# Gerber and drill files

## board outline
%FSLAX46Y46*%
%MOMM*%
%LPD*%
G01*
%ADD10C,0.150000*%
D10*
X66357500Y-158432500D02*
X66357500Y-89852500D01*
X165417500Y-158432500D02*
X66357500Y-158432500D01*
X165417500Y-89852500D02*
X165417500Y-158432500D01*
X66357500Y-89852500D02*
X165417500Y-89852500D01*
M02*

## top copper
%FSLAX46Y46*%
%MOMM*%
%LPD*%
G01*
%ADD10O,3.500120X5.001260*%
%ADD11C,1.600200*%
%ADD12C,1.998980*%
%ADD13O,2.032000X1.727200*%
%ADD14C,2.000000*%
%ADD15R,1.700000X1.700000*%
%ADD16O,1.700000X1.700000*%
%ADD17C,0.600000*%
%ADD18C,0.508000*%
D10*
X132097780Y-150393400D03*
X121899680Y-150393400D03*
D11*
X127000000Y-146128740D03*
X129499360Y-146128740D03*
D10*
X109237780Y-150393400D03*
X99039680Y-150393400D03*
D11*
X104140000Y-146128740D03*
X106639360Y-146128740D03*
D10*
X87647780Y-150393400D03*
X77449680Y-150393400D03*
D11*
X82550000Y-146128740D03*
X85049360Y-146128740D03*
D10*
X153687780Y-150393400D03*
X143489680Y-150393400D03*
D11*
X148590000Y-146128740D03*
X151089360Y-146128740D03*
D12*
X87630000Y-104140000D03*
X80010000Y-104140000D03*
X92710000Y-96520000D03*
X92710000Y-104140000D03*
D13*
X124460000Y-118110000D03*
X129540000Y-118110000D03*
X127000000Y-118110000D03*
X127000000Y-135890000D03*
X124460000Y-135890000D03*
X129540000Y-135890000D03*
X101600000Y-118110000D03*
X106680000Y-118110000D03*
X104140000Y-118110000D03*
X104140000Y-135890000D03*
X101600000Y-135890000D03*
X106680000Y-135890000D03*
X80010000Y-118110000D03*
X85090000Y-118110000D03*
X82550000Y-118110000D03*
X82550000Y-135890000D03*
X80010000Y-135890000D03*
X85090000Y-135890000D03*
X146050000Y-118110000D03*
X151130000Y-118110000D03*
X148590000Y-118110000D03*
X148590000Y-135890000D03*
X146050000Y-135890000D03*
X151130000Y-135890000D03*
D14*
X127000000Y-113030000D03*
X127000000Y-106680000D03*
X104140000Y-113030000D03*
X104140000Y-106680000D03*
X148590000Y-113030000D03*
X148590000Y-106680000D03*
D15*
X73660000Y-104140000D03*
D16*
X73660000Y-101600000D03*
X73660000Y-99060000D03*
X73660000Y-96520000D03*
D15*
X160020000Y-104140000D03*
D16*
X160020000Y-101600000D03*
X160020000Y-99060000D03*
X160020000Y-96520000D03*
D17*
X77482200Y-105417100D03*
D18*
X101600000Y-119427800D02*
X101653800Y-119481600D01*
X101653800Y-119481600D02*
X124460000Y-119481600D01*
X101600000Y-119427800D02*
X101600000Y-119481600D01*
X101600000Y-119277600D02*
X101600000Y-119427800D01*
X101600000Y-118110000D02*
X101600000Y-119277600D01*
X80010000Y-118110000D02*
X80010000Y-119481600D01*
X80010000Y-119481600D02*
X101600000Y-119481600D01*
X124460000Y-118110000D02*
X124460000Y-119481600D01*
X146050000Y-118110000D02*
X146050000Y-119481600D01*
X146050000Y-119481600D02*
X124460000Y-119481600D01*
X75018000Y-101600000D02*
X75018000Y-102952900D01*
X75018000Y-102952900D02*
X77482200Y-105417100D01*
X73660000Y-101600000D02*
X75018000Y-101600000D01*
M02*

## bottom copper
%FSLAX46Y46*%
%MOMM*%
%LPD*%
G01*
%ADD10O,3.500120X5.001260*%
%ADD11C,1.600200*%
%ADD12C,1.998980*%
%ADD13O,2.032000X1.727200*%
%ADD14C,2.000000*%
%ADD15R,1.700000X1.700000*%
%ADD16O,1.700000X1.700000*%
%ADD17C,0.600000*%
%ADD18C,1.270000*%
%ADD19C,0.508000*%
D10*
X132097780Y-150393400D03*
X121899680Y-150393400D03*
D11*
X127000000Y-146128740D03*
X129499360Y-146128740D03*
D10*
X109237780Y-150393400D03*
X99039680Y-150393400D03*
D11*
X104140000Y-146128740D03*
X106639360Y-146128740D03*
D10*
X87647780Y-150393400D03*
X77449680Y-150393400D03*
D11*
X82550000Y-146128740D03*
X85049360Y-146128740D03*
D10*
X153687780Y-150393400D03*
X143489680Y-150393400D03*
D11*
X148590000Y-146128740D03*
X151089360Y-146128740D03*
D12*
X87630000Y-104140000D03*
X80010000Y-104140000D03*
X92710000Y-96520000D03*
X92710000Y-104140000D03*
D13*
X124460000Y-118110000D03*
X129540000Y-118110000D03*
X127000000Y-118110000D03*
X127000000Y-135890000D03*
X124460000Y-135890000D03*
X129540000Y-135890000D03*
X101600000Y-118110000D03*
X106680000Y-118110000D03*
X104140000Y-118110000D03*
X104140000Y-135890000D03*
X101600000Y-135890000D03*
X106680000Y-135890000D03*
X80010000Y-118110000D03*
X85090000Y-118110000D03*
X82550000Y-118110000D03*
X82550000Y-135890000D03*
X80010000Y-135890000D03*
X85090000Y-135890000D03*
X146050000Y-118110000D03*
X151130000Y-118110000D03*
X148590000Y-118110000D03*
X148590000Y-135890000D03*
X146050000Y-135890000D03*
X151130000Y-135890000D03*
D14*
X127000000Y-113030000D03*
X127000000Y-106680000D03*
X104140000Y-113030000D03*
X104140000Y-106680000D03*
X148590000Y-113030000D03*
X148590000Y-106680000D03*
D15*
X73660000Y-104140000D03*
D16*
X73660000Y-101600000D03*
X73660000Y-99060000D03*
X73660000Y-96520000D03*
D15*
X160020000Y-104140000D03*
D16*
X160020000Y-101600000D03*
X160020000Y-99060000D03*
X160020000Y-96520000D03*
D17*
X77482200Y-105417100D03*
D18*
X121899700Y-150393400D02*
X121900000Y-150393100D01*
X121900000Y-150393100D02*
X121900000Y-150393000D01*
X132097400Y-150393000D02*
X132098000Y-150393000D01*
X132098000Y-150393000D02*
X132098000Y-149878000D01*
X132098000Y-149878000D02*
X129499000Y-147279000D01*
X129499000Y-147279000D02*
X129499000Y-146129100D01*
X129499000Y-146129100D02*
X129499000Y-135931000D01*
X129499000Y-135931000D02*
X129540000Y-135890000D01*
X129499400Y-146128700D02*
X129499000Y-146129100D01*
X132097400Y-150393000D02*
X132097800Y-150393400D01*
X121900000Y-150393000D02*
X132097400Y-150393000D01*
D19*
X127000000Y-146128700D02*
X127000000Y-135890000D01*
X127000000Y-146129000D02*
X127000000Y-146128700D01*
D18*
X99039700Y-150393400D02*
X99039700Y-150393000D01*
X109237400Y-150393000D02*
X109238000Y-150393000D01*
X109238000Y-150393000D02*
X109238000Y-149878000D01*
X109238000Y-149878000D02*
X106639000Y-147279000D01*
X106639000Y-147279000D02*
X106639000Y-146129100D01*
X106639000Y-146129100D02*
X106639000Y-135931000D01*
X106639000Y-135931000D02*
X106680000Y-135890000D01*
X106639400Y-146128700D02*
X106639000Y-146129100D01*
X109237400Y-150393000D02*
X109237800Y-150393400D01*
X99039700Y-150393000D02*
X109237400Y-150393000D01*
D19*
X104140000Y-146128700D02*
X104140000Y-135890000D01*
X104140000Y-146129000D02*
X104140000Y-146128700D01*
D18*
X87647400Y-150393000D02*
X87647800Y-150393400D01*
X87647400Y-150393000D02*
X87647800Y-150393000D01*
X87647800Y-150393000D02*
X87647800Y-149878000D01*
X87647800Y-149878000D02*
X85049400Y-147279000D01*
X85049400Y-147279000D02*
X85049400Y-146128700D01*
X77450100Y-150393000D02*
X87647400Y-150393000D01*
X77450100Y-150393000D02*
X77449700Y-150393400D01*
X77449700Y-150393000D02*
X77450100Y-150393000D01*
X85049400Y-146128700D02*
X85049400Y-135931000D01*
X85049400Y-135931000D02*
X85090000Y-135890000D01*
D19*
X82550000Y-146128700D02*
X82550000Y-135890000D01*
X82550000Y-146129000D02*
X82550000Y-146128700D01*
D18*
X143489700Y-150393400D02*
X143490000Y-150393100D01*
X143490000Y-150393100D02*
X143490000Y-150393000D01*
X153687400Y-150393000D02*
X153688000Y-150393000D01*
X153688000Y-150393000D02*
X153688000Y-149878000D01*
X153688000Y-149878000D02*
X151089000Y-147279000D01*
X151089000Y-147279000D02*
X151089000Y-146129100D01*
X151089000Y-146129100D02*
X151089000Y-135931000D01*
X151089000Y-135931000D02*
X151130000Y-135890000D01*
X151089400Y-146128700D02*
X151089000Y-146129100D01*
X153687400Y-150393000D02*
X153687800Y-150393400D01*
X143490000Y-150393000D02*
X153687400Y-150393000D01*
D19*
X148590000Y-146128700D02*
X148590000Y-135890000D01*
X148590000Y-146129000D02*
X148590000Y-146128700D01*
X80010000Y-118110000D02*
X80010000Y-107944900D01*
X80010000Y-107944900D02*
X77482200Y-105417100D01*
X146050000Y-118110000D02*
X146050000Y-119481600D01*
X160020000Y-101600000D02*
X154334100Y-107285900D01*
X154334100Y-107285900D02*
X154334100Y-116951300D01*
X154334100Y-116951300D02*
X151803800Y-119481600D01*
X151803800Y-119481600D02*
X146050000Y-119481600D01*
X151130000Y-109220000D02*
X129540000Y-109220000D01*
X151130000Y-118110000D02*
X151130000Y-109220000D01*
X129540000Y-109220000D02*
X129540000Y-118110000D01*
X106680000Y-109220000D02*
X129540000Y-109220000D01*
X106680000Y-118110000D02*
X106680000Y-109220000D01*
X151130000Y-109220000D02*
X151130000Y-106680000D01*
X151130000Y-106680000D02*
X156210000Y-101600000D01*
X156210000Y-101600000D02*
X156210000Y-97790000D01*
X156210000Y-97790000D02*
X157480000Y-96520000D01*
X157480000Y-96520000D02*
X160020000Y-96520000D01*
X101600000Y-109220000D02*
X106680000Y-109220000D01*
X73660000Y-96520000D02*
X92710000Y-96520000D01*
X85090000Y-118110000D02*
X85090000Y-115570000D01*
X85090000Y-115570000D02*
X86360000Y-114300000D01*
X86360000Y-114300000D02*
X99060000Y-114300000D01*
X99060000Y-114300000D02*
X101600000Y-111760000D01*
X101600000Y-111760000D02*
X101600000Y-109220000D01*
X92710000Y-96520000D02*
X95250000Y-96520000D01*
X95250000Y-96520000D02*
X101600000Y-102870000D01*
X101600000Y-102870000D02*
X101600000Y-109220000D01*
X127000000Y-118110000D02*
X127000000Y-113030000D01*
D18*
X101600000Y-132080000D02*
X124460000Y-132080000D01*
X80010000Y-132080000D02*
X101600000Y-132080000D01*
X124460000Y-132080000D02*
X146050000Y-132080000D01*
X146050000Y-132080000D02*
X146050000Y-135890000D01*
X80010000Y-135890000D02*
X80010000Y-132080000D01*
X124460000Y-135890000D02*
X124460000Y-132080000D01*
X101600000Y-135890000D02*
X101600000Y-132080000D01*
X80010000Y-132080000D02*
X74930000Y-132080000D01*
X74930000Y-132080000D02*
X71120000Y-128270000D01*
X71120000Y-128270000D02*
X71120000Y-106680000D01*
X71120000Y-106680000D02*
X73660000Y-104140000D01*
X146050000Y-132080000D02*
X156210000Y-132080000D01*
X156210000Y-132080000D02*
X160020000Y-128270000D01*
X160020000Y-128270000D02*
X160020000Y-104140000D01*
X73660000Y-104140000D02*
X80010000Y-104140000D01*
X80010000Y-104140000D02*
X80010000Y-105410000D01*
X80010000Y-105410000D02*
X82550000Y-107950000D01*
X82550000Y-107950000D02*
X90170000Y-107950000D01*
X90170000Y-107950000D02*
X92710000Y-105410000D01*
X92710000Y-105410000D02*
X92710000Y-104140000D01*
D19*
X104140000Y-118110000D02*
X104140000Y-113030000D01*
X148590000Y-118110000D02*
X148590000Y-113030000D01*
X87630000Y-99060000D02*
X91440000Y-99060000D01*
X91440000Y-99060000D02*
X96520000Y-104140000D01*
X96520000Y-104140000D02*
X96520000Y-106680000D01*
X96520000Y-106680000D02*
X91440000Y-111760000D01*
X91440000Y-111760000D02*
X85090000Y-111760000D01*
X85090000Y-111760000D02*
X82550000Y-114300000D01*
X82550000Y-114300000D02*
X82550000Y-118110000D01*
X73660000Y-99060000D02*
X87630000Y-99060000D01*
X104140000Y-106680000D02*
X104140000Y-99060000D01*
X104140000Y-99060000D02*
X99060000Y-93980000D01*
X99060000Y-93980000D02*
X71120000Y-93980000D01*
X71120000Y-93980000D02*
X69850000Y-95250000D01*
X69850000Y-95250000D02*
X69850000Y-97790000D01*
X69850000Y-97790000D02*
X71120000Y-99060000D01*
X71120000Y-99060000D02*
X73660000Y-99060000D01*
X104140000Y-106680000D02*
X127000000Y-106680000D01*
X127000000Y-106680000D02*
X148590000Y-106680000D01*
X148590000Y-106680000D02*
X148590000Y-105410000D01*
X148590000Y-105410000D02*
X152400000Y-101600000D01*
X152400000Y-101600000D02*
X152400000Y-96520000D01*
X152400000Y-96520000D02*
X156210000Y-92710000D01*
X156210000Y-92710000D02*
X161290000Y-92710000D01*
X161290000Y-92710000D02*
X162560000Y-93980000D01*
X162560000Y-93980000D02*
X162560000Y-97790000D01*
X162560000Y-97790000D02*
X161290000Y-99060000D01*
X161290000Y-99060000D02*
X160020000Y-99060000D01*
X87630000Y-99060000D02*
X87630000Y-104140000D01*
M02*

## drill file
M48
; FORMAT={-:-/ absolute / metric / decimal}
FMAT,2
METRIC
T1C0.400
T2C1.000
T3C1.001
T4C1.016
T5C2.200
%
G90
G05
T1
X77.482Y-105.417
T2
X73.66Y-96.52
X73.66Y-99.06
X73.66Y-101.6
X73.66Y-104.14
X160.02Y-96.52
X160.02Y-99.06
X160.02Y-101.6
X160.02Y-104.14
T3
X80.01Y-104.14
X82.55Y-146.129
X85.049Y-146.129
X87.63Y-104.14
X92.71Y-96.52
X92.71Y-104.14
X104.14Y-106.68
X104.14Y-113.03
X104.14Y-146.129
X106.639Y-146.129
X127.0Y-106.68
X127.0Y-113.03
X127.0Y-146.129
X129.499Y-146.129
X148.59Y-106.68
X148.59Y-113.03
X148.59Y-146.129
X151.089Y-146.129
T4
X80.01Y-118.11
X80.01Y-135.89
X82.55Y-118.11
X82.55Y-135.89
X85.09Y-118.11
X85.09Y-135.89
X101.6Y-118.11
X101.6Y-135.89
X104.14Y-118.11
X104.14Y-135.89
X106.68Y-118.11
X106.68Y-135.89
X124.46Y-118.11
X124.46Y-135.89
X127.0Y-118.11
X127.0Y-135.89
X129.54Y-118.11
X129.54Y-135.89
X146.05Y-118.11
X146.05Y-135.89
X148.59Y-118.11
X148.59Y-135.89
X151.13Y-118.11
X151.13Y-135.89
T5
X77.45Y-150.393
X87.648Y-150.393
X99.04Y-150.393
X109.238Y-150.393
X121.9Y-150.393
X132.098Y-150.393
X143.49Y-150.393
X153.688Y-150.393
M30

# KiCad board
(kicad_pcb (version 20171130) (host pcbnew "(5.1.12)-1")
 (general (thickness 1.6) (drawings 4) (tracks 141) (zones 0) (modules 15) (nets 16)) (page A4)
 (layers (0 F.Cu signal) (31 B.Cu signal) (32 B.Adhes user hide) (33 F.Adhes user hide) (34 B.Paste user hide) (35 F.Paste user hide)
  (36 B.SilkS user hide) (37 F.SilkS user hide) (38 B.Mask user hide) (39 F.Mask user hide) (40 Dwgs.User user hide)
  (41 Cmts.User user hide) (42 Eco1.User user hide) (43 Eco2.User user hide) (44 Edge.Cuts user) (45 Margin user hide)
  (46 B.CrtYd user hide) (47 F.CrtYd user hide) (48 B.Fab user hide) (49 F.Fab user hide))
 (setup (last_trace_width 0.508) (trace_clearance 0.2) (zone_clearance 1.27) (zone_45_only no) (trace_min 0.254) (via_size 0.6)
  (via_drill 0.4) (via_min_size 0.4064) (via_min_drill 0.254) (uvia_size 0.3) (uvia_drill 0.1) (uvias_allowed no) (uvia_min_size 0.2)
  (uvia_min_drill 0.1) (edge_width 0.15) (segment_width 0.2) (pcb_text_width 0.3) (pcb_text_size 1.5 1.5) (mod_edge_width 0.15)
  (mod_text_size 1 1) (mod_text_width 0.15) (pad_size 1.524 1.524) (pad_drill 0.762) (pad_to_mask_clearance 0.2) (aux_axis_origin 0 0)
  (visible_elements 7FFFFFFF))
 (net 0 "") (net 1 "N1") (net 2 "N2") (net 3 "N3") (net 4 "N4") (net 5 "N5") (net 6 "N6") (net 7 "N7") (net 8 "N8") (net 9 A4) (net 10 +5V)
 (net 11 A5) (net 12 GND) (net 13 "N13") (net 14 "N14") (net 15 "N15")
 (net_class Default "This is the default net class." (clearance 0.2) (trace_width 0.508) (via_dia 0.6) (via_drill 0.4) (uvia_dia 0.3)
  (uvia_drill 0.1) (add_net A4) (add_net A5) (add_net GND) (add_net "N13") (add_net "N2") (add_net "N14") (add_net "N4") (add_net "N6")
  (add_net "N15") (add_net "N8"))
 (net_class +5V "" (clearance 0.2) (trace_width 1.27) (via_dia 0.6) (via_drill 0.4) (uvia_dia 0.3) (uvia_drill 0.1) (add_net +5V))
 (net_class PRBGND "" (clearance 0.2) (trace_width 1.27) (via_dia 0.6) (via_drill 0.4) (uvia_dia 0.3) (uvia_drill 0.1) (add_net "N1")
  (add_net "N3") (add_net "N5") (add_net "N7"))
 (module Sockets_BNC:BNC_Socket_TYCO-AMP (layer F.Cu) (at 127 151.13 180)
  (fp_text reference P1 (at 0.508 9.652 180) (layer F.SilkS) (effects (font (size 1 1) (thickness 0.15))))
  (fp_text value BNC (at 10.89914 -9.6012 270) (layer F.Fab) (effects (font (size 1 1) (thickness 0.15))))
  (pad 2 thru_hole oval (at -5.09778 0.7366 180) (size 3.50012 5.00126) (drill 2.19964) (layers *.Cu *.Mask) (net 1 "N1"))
  (pad 2 thru_hole oval (at 5.10032 0.7366 180) (size 3.50012 5.00126) (drill 2.19964) (layers *.Cu *.Mask) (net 1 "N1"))
  (pad 1 thru_hole circle (at 0 5.00126 180) (size 1.6002 1.6002) (drill 1.00076) (layers *.Cu *.Mask) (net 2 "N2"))
  (pad 2 thru_hole circle (at -2.49936 5.00126 180) (size 1.6002 1.6002) (drill 1.00076) (layers *.Cu *.Mask) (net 1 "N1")))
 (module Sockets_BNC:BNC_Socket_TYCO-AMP (layer F.Cu) (at 104.14 151.13 180)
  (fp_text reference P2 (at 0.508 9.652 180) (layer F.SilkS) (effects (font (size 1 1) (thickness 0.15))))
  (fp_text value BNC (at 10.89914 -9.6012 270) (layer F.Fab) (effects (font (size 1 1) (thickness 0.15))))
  (pad 2 thru_hole oval (at -5.09778 0.7366 180) (size 3.50012 5.00126) (drill 2.19964) (layers *.Cu *.Mask) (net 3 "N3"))
  (pad 2 thru_hole oval (at 5.10032 0.7366 180) (size 3.50012 5.00126) (drill 2.19964) (layers *.Cu *.Mask) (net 3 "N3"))
  (pad 1 thru_hole circle (at 0 5.00126 180) (size 1.6002 1.6002) (drill 1.00076) (layers *.Cu *.Mask) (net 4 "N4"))
  (pad 2 thru_hole circle (at -2.49936 5.00126 180) (size 1.6002 1.6002) (drill 1.00076) (layers *.Cu *.Mask) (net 3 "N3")))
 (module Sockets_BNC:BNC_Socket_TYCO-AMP (layer F.Cu) (at 82.55 151.13 180)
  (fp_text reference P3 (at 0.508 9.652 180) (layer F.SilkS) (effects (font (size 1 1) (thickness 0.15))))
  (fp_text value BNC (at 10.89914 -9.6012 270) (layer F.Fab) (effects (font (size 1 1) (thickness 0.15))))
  (pad 2 thru_hole oval (at -5.09778 0.7366 180) (size 3.50012 5.00126) (drill 2.19964) (layers *.Cu *.Mask) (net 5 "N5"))
  (pad 2 thru_hole oval (at 5.10032 0.7366 180) (size 3.50012 5.00126) (drill 2.19964) (layers *.Cu *.Mask) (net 5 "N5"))
  (pad 1 thru_hole circle (at 0 5.00126 180) (size 1.6002 1.6002) (drill 1.00076) (layers *.Cu *.Mask) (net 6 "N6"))
  (pad 2 thru_hole circle (at -2.49936 5.00126 180) (size 1.6002 1.6002) (drill 1.00076) (layers *.Cu *.Mask) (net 5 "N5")))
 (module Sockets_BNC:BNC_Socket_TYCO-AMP (layer F.Cu) (at 148.59 151.13 180)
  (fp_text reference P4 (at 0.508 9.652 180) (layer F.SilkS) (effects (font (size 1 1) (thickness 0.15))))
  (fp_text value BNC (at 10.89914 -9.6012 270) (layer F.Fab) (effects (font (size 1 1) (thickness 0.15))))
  (pad 2 thru_hole oval (at -5.09778 0.7366 180) (size 3.50012 5.00126) (drill 2.19964) (layers *.Cu *.Mask) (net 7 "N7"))
  (pad 2 thru_hole oval (at 5.10032 0.7366 180) (size 3.50012 5.00126) (drill 2.19964) (layers *.Cu *.Mask) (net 7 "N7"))
  (pad 1 thru_hole circle (at 0 5.00126 180) (size 1.6002 1.6002) (drill 1.00076) (layers *.Cu *.Mask) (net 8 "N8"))
  (pad 2 thru_hole circle (at -2.49936 5.00126 180) (size 1.6002 1.6002) (drill 1.00076) (layers *.Cu *.Mask) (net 7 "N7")))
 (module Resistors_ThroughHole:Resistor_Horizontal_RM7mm (layer F.Cu) (at 87.63 104.14 180)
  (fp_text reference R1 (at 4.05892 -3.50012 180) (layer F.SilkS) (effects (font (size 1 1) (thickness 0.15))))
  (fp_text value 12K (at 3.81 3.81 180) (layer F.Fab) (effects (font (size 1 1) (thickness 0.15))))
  (pad 1 thru_hole circle (at 0 0 180) (size 1.99898 1.99898) (drill 1.00076) (layers *.Cu *.SilkS *.Mask) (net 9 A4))
  (pad 2 thru_hole circle (at 7.62 0 180) (size 1.99898 1.99898) (drill 1.00076) (layers *.Cu *.SilkS *.Mask) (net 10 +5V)))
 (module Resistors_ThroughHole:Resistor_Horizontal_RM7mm (layer F.Cu) (at 92.71 96.52 270)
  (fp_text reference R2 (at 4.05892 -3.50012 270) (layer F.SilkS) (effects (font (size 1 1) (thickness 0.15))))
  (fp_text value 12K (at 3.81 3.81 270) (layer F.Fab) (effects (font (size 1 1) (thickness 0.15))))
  (pad 1 thru_hole circle (at 0 0 270) (size 1.99898 1.99898) (drill 1.00076) (layers *.Cu *.SilkS *.Mask) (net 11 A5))
  (pad 2 thru_hole circle (at 7.62 0 270) (size 1.99898 1.99898) (drill 1.00076) (layers *.Cu *.SilkS *.Mask) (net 10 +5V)))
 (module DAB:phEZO (layer F.Cu) (at 127 127)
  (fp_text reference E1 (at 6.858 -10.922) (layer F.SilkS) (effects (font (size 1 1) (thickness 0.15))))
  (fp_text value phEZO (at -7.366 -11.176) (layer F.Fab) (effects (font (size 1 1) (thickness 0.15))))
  (pad 1 thru_hole oval (at -2.54 -8.89) (size 2.032 1.7272) (drill 1.016) (layers *.Cu *.Mask) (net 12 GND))
  (pad 3 thru_hole oval (at 2.54 -8.89) (size 2.032 1.7272) (drill 1.016) (layers *.Cu *.Mask) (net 11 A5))
  (pad 2 thru_hole oval (at 0 -8.89) (size 2.032 1.7272) (drill 1.016) (layers *.Cu *.Mask) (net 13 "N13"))
  (pad 5 thru_hole oval (at 0 8.89) (size 2.032 1.7272) (drill 1.016) (layers *.Cu *.Mask) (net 2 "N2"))
  (pad 6 thru_hole oval (at -2.54 8.89) (size 2.032 1.7272) (drill 1.016) (layers *.Cu *.Mask) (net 10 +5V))
  (pad 4 thru_hole oval (at 2.54 8.89) (size 2.032 1.7272) (drill 1.016) (layers *.Cu *.Mask) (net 1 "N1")))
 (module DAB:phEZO (layer F.Cu) (at 104.14 127)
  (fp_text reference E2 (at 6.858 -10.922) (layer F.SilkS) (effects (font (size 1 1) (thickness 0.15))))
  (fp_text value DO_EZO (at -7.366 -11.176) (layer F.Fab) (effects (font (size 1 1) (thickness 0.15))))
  (pad 1 thru_hole oval (at -2.54 -8.89) (size 2.032 1.7272) (drill 1.016) (layers *.Cu *.Mask) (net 12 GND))
  (pad 3 thru_hole oval (at 2.54 -8.89) (size 2.032 1.7272) (drill 1.016) (layers *.Cu *.Mask) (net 11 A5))
  (pad 2 thru_hole oval (at 0 -8.89) (size 2.032 1.7272) (drill 1.016) (layers *.Cu *.Mask) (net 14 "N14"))
  (pad 5 thru_hole oval (at 0 8.89) (size 2.032 1.7272) (drill 1.016) (layers *.Cu *.Mask) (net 4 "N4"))
  (pad 6 thru_hole oval (at -2.54 8.89) (size 2.032 1.7272) (drill 1.016) (layers *.Cu *.Mask) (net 10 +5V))
  (pad 4 thru_hole oval (at 2.54 8.89) (size 2.032 1.7272) (drill 1.016) (layers *.Cu *.Mask) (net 3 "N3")))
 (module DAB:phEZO (layer F.Cu) (at 82.55 127)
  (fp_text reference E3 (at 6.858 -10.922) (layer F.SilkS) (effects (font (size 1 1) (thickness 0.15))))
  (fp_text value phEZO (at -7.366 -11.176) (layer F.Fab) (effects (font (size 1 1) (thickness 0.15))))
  (pad 1 thru_hole oval (at -2.54 -8.89) (size 2.032 1.7272) (drill 1.016) (layers *.Cu *.Mask) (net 12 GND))
  (pad 3 thru_hole oval (at 2.54 -8.89) (size 2.032 1.7272) (drill 1.016) (layers *.Cu *.Mask) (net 11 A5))
  (pad 2 thru_hole oval (at 0 -8.89) (size 2.032 1.7272) (drill 1.016) (layers *.Cu *.Mask) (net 9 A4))
  (pad 5 thru_hole oval (at 0 8.89) (size 2.032 1.7272) (drill 1.016) (layers *.Cu *.Mask) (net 6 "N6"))
  (pad 6 thru_hole oval (at -2.54 8.89) (size 2.032 1.7272) (drill 1.016) (layers *.Cu *.Mask) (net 10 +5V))
  (pad 4 thru_hole oval (at 2.54 8.89) (size 2.032 1.7272) (drill 1.016) (layers *.Cu *.Mask) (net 5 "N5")))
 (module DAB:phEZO (layer F.Cu) (at 148.59 127)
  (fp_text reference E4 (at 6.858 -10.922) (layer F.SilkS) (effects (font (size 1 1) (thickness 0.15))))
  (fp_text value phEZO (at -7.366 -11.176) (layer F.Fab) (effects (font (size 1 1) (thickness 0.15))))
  (pad 1 thru_hole oval (at -2.54 -8.89) (size 2.032 1.7272) (drill 1.016) (layers *.Cu *.Mask) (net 12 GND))
  (pad 3 thru_hole oval (at 2.54 -8.89) (size 2.032 1.7272) (drill 1.016) (layers *.Cu *.Mask) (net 11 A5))
  (pad 2 thru_hole oval (at 0 -8.89) (size 2.032 1.7272) (drill 1.016) (layers *.Cu *.Mask) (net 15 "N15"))
  (pad 5 thru_hole oval (at 0 8.89) (size 2.032 1.7272) (drill 1.016) (layers *.Cu *.Mask) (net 8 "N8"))
  (pad 6 thru_hole oval (at -2.54 8.89) (size 2.032 1.7272) (drill 1.016) (layers *.Cu *.Mask) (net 10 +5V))
  (pad 4 thru_hole oval (at 2.54 8.89) (size 2.032 1.7272) (drill 1.016) (layers *.Cu *.Mask) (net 7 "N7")))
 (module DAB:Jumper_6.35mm (layer F.Cu) (at 127 113.03 90)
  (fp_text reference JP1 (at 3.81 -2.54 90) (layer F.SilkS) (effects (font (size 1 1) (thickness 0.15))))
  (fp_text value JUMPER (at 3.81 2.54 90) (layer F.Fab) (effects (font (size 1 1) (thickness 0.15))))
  (pad 1 thru_hole circle (at 0 0 90) (size 2 2) (drill 1.00076) (layers *.Cu *.Mask) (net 13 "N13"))
  (pad 2 thru_hole circle (at 6.35 0 90) (size 2 2) (drill 1.00076) (layers *.Cu *.Mask) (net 9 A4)))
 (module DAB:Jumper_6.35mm (layer F.Cu) (at 104.14 113.03 90)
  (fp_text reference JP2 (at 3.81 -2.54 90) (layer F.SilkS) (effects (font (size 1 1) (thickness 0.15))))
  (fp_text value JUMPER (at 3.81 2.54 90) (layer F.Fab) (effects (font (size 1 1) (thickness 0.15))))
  (pad 1 thru_hole circle (at 0 0 90) (size 2 2) (drill 1.00076) (layers *.Cu *.Mask) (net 14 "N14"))
  (pad 2 thru_hole circle (at 6.35 0 90) (size 2 2) (drill 1.00076) (layers *.Cu *.Mask) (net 9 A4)))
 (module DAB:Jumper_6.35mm (layer F.Cu) (at 148.59 113.03 90)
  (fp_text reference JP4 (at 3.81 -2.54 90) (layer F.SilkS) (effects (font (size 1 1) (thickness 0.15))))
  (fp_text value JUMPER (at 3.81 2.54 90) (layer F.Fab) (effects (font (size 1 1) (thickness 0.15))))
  (pad 1 thru_hole circle (at 0 0 90) (size 2 2) (drill 1.00076) (layers *.Cu *.Mask) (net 15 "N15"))
  (pad 2 thru_hole circle (at 6.35 0 90) (size 2 2) (drill 1.00076) (layers *.Cu *.Mask) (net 9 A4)))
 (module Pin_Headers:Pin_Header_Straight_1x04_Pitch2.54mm (layer F.Cu) (at 73.66 104.14 180)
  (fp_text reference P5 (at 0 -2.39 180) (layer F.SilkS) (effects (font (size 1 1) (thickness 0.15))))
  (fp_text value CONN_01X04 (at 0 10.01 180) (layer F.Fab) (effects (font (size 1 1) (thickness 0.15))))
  (pad 1 thru_hole rect (at 0 0 180) (size 1.7 1.7) (drill 1) (layers *.Cu *.Mask) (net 10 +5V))
  (pad 2 thru_hole oval (at 0 2.54 180) (size 1.7 1.7) (drill 1) (layers *.Cu *.Mask) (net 12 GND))
  (pad 3 thru_hole oval (at 0 5.08 180) (size 1.7 1.7) (drill 1) (layers *.Cu *.Mask) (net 9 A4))
  (pad 4 thru_hole oval (at 0 7.62 180) (size 1.7 1.7) (drill 1) (layers *.Cu *.Mask) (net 11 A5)))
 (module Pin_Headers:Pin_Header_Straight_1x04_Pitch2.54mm (layer F.Cu) (at 160.02 104.14 180)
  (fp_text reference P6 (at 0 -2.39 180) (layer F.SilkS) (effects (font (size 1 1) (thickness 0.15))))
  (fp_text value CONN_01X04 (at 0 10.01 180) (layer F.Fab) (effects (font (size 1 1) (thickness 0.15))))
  (pad 1 thru_hole rect (at 0 0 180) (size 1.7 1.7) (drill 1) (layers *.Cu *.Mask) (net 10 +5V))
  (pad 2 thru_hole oval (at 0 2.54 180) (size 1.7 1.7) (drill 1) (layers *.Cu *.Mask) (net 12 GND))
  (pad 3 thru_hole oval (at 0 5.08 180) (size 1.7 1.7) (drill 1) (layers *.Cu *.Mask) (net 9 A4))
  (pad 4 thru_hole oval (at 0 7.62 180) (size 1.7 1.7) (drill 1) (layers *.Cu *.Mask) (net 11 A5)))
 (gr_line (start 66.3575 158.4325) (end 66.3575 89.8525) (angle 90) (layer Edge.Cuts) (width 0.15))
 (gr_line (start 165.4175 158.4325) (end 66.3575 158.4325) (angle 90) (layer Edge.Cuts) (width 0.15))
 (gr_line (start 165.4175 89.8525) (end 165.4175 158.4325) (angle 90) (layer Edge.Cuts) (width 0.15))
 (gr_line (start 66.3575 89.8525) (end 165.4175 89.8525) (angle 90) (layer Edge.Cuts) (width 0.15))
 (segment (start 121.8997 150.3934) (end 121.9 150.3931) (width 1.27) (layer B.Cu) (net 1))
 (segment (start 121.9 150.3931) (end 121.9 150.393) (width 1.27) (layer B.Cu) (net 1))
 (segment (start 132.0974 150.393) (end 132.098 150.393) (width 1.27) (layer B.Cu) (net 1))
 (segment (start 132.098 150.393) (end 132.098 149.878) (width 1.27) (layer B.Cu) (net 1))
 (segment (start 132.098 149.878) (end 129.499 147.279) (width 1.27) (layer B.Cu) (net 1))
 (segment (start 129.499 147.279) (end 129.499 146.1291) (width 1.27) (layer B.Cu) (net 1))
 (segment (start 129.499 146.1291) (end 129.499 135.931) (width 1.27) (layer B.Cu) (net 1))
 (segment (start 129.499 135.931) (end 129.54 135.89) (width 1.27) (layer B.Cu) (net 1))
 (segment (start 129.4994 146.1287) (end 129.499 146.1291) (width 1.27) (layer B.Cu) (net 1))
 (segment (start 132.0974 150.393) (end 132.0978 150.3934) (width 1.27) (layer B.Cu) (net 1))
 (segment (start 121.9 150.393) (end 132.0974 150.393) (width 1.27) (layer B.Cu) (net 1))
 (segment (start 127 146.1287) (end 127 135.89) (width 0.508) (layer B.Cu) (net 2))
 (segment (start 127 146.129) (end 127 146.1287) (width 0.508) (layer B.Cu) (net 2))
 (segment (start 99.0397 150.3934) (end 99.0397 150.393) (width 1.27) (layer B.Cu) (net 3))
 (segment (start 109.2374 150.393) (end 109.238 150.393) (width 1.27) (layer B.Cu) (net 3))
 (segment (start 109.238 150.393) (end 109.238 149.878) (width 1.27) (layer B.Cu) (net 3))
 (segment (start 109.238 149.878) (end 106.639 147.279) (width 1.27) (layer B.Cu) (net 3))
 (segment (start 106.639 147.279) (end 106.639 146.1291) (width 1.27) (layer B.Cu) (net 3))
 (segment (start 106.639 146.1291) (end 106.639 135.931) (width 1.27) (layer B.Cu) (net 3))
 (segment (start 106.639 135.931) (end 106.68 135.89) (width 1.27) (layer B.Cu) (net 3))
 (segment (start 106.6394 146.1287) (end 106.639 146.1291) (width 1.27) (layer B.Cu) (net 3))
 (segment (start 109.2374 150.393) (end 109.2378 150.3934) (width 1.27) (layer B.Cu) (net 3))
 (segment (start 99.0397 150.393) (end 109.2374 150.393) (width 1.27) (layer B.Cu) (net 3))
 (segment (start 104.14 146.1287) (end 104.14 135.89) (width 0.508) (layer B.Cu) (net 4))
 (segment (start 104.14 146.129) (end 104.14 146.1287) (width 0.508) (layer B.Cu) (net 4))
 (segment (start 87.6474 150.393) (end 87.6478 150.3934) (width 1.27) (layer B.Cu) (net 5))
 (segment (start 87.6474 150.393) (end 87.6478 150.393) (width 1.27) (layer B.Cu) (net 5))
 (segment (start 87.6478 150.393) (end 87.6478 149.878) (width 1.27) (layer B.Cu) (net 5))
 (segment (start 87.6478 149.878) (end 85.0494 147.279) (width 1.27) (layer B.Cu) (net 5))
 (segment (start 85.0494 147.279) (end 85.0494 146.1287) (width 1.27) (layer B.Cu) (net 5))
 (segment (start 77.4501 150.393) (end 87.6474 150.393) (width 1.27) (layer B.Cu) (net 5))
 (segment (start 77.4501 150.393) (end 77.4497 150.3934) (width 1.27) (layer B.Cu) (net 5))
 (segment (start 77.4497 150.393) (end 77.4501 150.393) (width 1.27) (layer B.Cu) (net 5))
 (segment (start 85.0494 146.1287) (end 85.0494 135.931) (width 1.27) (layer B.Cu) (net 5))
 (segment (start 85.0494 135.931) (end 85.09 135.89) (width 1.27) (layer B.Cu) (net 5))
 (segment (start 82.55 146.1287) (end 82.55 135.89) (width 0.508) (layer B.Cu) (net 6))
 (segment (start 82.55 146.129) (end 82.55 146.1287) (width 0.508) (layer B.Cu) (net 6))
 (segment (start 143.4897 150.3934) (end 143.49 150.3931) (width 1.27) (layer B.Cu) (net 7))
 (segment (start 143.49 150.3931) (end 143.49 150.393) (width 1.27) (layer B.Cu) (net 7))
 (segment (start 153.6874 150.393) (end 153.688 150.393) (width 1.27) (layer B.Cu) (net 7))
 (segment (start 153.688 150.393) (end 153.688 149.878) (width 1.27) (layer B.Cu) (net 7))
 (segment (start 153.688 149.878) (end 151.089 147.279) (width 1.27) (layer B.Cu) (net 7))
 (segment (start 151.089 147.279) (end 151.089 146.1291) (width 1.27) (layer B.Cu) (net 7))
 (segment (start 151.089 146.1291) (end 151.089 135.931) (width 1.27) (layer B.Cu) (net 7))
 (segment (start 151.089 135.931) (end 151.13 135.89) (width 1.27) (layer B.Cu) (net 7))
 (segment (start 151.0894 146.1287) (end 151.089 146.1291) (width 1.27) (layer B.Cu) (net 7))
 (segment (start 153.6874 150.393) (end 153.6878 150.3934) (width 1.27) (layer B.Cu) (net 7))
 (segment (start 143.49 150.393) (end 153.6874 150.393) (width 1.27) (layer B.Cu) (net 7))
 (segment (start 148.59 146.1287) (end 148.59 135.89) (width 0.508) (layer B.Cu) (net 8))
 (segment (start 148.59 146.129) (end 148.59 146.1287) (width 0.508) (layer B.Cu) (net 8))
 (segment (start 101.6 119.4278) (end 101.6538 119.4816) (width 0.508) (layer F.Cu) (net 12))
 (segment (start 101.6538 119.4816) (end 124.46 119.4816) (width 0.508) (layer F.Cu) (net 12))
 (segment (start 101.6 119.4278) (end 101.6 119.4816) (width 0.508) (layer F.Cu) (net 12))
 (segment (start 101.6 119.2776) (end 101.6 119.4278) (width 0.508) (layer F.Cu) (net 12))
 (segment (start 101.6 118.11) (end 101.6 119.2776) (width 0.508) (layer F.Cu) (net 12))
 (segment (start 80.01 118.11) (end 80.01 119.4816) (width 0.508) (layer F.Cu) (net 12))
 (segment (start 80.01 119.4816) (end 101.6 119.4816) (width 0.508) (layer F.Cu) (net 12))
 (segment (start 124.46 118.11) (end 124.46 119.4816) (width 0.508) (layer F.Cu) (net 12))
 (segment (start 146.05 118.11) (end 146.05 119.4816) (width 0.508) (layer F.Cu) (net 12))
 (segment (start 146.05 119.4816) (end 124.46 119.4816) (width 0.508) (layer F.Cu) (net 12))
 (segment (start 75.018 101.6) (end 75.018 102.9529) (width 0.508) (layer F.Cu) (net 12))
 (segment (start 75.018 102.9529) (end 77.4822 105.4171) (width 0.508) (layer F.Cu) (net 12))
 (segment (start 80.01 118.11) (end 80.01 107.9449) (width 0.508) (layer B.Cu) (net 12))
 (segment (start 80.01 107.9449) (end 77.4822 105.4171) (width 0.508) (layer B.Cu) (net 12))
 (segment (start 73.66 101.6) (end 75.018 101.6) (width 0.508) (layer F.Cu) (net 12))
 (segment (start 146.05 118.11) (end 146.05 119.4816) (width 0.508) (layer B.Cu) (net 12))
 (segment (start 160.02 101.6) (end 154.3341 107.2859) (width 0.508) (layer B.Cu) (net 12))
 (segment (start 154.3341 107.2859) (end 154.3341 116.9513) (width 0.508) (layer B.Cu) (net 12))
 (segment (start 154.3341 116.9513) (end 151.8038 119.4816) (width 0.508) (layer B.Cu) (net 12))
 (segment (start 151.8038 119.4816) (end 146.05 119.4816) (width 0.508) (layer B.Cu) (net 12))
 (via (at 77.4822 105.4171) (size 0.6) (layers F.Cu B.Cu) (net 12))
 (segment (start 151.13 109.22) (end 129.54 109.22) (width 0.508) (layer B.Cu) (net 11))
 (segment (start 151.13 118.11) (end 151.13 109.22) (width 0.508) (layer B.Cu) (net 11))
 (segment (start 129.54 109.22) (end 129.54 118.11) (width 0.508) (layer B.Cu) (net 11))
 (segment (start 106.68 109.22) (end 129.54 109.22) (width 0.508) (layer B.Cu) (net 11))
 (segment (start 106.68 118.11) (end 106.68 109.22) (width 0.508) (layer B.Cu) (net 11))
 (segment (start 151.13 109.22) (end 151.13 106.68) (width 0.508) (layer B.Cu) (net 11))
 (segment (start 151.13 106.68) (end 156.21 101.6) (width 0.508) (layer B.Cu) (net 11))
 (segment (start 156.21 101.6) (end 156.21 97.79) (width 0.508) (layer B.Cu) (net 11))
 (segment (start 156.21 97.79) (end 157.48 96.52) (width 0.508) (layer B.Cu) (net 11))
 (segment (start 157.48 96.52) (end 160.02 96.52) (width 0.508) (layer B.Cu) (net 11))
 (segment (start 101.6 109.22) (end 106.68 109.22) (width 0.508) (layer B.Cu) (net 11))
 (segment (start 73.66 96.52) (end 92.71 96.52) (width 0.508) (layer B.Cu) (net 11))
 (segment (start 85.09 118.11) (end 85.09 115.57) (width 0.508) (layer B.Cu) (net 11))
 (segment (start 85.09 115.57) (end 86.36 114.3) (width 0.508) (layer B.Cu) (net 11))
 (segment (start 86.36 114.3) (end 99.06 114.3) (width 0.508) (layer B.Cu) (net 11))
 (segment (start 99.06 114.3) (end 101.6 111.76) (width 0.508) (layer B.Cu) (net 11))
 (segment (start 101.6 111.76) (end 101.6 109.22) (width 0.508) (layer B.Cu) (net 11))
 (segment (start 92.71 96.52) (end 95.25 96.52) (width 0.508) (layer B.Cu) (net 11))
 (segment (start 95.25 96.52) (end 101.6 102.87) (width 0.508) (layer B.Cu) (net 11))
 (segment (start 101.6 102.87) (end 101.6 109.22) (width 0.508) (layer B.Cu) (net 11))
 (segment (start 127 118.11) (end 127 113.03) (width 0.508) (layer B.Cu) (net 13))
 (segment (start 101.6 132.08) (end 124.46 132.08) (width 1.27) (layer B.Cu) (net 10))
 (segment (start 80.01 132.08) (end 101.6 132.08) (width 1.27) (layer B.Cu) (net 10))
 (segment (start 124.46 132.08) (end 146.05 132.08) (width 1.27) (layer B.Cu) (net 10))
 (segment (start 146.05 132.08) (end 146.05 135.89) (width 1.27) (layer B.Cu) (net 10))
 (segment (start 80.01 135.89) (end 80.01 132.08) (width 1.27) (layer B.Cu) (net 10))
 (segment (start 124.46 135.89) (end 124.46 132.08) (width 1.27) (layer B.Cu) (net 10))
 (segment (start 101.6 135.89) (end 101.6 132.08) (width 1.27) (layer B.Cu) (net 10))
 (segment (start 80.01 132.08) (end 74.93 132.08) (width 1.27) (layer B.Cu) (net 10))
 (segment (start 74.93 132.08) (end 71.12 128.27) (width 1.27) (layer B.Cu) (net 10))
 (segment (start 71.12 128.27) (end 71.12 106.68) (width 1.27) (layer B.Cu) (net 10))
 (segment (start 71.12 106.68) (end 73.66 104.14) (width 1.27) (layer B.Cu) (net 10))
 (segment (start 146.05 132.08) (end 156.21 132.08) (width 1.27) (layer B.Cu) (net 10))
 (segment (start 156.21 132.08) (end 160.02 128.27) (width 1.27) (layer B.Cu) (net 10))
 (segment (start 160.02 128.27) (end 160.02 104.14) (width 1.27) (layer B.Cu) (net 10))
 (segment (start 73.66 104.14) (end 80.01 104.14) (width 1.27) (layer B.Cu) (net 10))
 (segment (start 80.01 104.14) (end 80.01 105.41) (width 1.27) (layer B.Cu) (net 10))
 (segment (start 80.01 105.41) (end 82.55 107.95) (width 1.27) (layer B.Cu) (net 10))
 (segment (start 82.55 107.95) (end 90.17 107.95) (width 1.27) (layer B.Cu) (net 10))
 (segment (start 90.17 107.95) (end 92.71 105.41) (width 1.27) (layer B.Cu) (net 10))
 (segment (start 92.71 105.41) (end 92.71 104.14) (width 1.27) (layer B.Cu) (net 10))
 (segment (start 104.14 118.11) (end 104.14 113.03) (width 0.508) (layer B.Cu) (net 14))
 (segment (start 148.59 118.11) (end 148.59 113.03) (width 0.508) (layer B.Cu) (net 15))
 (segment (start 87.63 99.06) (end 91.44 99.06) (width 0.508) (layer B.Cu) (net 9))
 (segment (start 91.44 99.06) (end 96.52 104.14) (width 0.508) (layer B.Cu) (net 9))
 (segment (start 96.52 104.14) (end 96.52 106.68) (width 0.508) (layer B.Cu) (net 9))
 (segment (start 96.52 106.68) (end 91.44 111.76) (width 0.508) (layer B.Cu) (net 9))
 (segment (start 91.44 111.76) (end 85.09 111.76) (width 0.508) (layer B.Cu) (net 9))
 (segment (start 85.09 111.76) (end 82.55 114.3) (width 0.508) (layer B.Cu) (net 9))
 (segment (start 82.55 114.3) (end 82.55 118.11) (width 0.508) (layer B.Cu) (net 9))
 (segment (start 73.66 99.06) (end 87.63 99.06) (width 0.508) (layer B.Cu) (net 9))
 (segment (start 104.14 106.68) (end 104.14 99.06) (width 0.508) (layer B.Cu) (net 9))
 (segment (start 104.14 99.06) (end 99.06 93.98) (width 0.508) (layer B.Cu) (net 9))
 (segment (start 99.06 93.98) (end 71.12 93.98) (width 0.508) (layer B.Cu) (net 9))
 (segment (start 71.12 93.98) (end 69.85 95.25) (width 0.508) (layer B.Cu) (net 9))
 (segment (start 69.85 95.25) (end 69.85 97.79) (width 0.508) (layer B.Cu) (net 9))
 (segment (start 69.85 97.79) (end 71.12 99.06) (width 0.508) (layer B.Cu) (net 9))
 (segment (start 71.12 99.06) (end 73.66 99.06) (width 0.508) (layer B.Cu) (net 9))
 (segment (start 104.14 106.68) (end 127 106.68) (width 0.508) (layer B.Cu) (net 9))
 (segment (start 127 106.68) (end 148.59 106.68) (width 0.508) (layer B.Cu) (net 9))
 (segment (start 148.59 106.68) (end 148.59 105.41) (width 0.508) (layer B.Cu) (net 9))
 (segment (start 148.59 105.41) (end 152.4 101.6) (width 0.508) (layer B.Cu) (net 9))
 (segment (start 152.4 101.6) (end 152.4 96.52) (width 0.508) (layer B.Cu) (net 9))
 (segment (start 152.4 96.52) (end 156.21 92.71) (width 0.508) (layer B.Cu) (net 9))
 (segment (start 156.21 92.71) (end 161.29 92.71) (width 0.508) (layer B.Cu) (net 9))
 (segment (start 161.29 92.71) (end 162.56 93.98) (width 0.508) (layer B.Cu) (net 9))
 (segment (start 162.56 93.98) (end 162.56 97.79) (width 0.508) (layer B.Cu) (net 9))
 (segment (start 162.56 97.79) (end 161.29 99.06) (width 0.508) (layer B.Cu) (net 9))
 (segment (start 161.29 99.06) (end 160.02 99.06) (width 0.508) (layer B.Cu) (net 9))
 (segment (start 87.63 99.06) (end 87.63 104.14) (width 0.508) (layer B.Cu) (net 9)))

